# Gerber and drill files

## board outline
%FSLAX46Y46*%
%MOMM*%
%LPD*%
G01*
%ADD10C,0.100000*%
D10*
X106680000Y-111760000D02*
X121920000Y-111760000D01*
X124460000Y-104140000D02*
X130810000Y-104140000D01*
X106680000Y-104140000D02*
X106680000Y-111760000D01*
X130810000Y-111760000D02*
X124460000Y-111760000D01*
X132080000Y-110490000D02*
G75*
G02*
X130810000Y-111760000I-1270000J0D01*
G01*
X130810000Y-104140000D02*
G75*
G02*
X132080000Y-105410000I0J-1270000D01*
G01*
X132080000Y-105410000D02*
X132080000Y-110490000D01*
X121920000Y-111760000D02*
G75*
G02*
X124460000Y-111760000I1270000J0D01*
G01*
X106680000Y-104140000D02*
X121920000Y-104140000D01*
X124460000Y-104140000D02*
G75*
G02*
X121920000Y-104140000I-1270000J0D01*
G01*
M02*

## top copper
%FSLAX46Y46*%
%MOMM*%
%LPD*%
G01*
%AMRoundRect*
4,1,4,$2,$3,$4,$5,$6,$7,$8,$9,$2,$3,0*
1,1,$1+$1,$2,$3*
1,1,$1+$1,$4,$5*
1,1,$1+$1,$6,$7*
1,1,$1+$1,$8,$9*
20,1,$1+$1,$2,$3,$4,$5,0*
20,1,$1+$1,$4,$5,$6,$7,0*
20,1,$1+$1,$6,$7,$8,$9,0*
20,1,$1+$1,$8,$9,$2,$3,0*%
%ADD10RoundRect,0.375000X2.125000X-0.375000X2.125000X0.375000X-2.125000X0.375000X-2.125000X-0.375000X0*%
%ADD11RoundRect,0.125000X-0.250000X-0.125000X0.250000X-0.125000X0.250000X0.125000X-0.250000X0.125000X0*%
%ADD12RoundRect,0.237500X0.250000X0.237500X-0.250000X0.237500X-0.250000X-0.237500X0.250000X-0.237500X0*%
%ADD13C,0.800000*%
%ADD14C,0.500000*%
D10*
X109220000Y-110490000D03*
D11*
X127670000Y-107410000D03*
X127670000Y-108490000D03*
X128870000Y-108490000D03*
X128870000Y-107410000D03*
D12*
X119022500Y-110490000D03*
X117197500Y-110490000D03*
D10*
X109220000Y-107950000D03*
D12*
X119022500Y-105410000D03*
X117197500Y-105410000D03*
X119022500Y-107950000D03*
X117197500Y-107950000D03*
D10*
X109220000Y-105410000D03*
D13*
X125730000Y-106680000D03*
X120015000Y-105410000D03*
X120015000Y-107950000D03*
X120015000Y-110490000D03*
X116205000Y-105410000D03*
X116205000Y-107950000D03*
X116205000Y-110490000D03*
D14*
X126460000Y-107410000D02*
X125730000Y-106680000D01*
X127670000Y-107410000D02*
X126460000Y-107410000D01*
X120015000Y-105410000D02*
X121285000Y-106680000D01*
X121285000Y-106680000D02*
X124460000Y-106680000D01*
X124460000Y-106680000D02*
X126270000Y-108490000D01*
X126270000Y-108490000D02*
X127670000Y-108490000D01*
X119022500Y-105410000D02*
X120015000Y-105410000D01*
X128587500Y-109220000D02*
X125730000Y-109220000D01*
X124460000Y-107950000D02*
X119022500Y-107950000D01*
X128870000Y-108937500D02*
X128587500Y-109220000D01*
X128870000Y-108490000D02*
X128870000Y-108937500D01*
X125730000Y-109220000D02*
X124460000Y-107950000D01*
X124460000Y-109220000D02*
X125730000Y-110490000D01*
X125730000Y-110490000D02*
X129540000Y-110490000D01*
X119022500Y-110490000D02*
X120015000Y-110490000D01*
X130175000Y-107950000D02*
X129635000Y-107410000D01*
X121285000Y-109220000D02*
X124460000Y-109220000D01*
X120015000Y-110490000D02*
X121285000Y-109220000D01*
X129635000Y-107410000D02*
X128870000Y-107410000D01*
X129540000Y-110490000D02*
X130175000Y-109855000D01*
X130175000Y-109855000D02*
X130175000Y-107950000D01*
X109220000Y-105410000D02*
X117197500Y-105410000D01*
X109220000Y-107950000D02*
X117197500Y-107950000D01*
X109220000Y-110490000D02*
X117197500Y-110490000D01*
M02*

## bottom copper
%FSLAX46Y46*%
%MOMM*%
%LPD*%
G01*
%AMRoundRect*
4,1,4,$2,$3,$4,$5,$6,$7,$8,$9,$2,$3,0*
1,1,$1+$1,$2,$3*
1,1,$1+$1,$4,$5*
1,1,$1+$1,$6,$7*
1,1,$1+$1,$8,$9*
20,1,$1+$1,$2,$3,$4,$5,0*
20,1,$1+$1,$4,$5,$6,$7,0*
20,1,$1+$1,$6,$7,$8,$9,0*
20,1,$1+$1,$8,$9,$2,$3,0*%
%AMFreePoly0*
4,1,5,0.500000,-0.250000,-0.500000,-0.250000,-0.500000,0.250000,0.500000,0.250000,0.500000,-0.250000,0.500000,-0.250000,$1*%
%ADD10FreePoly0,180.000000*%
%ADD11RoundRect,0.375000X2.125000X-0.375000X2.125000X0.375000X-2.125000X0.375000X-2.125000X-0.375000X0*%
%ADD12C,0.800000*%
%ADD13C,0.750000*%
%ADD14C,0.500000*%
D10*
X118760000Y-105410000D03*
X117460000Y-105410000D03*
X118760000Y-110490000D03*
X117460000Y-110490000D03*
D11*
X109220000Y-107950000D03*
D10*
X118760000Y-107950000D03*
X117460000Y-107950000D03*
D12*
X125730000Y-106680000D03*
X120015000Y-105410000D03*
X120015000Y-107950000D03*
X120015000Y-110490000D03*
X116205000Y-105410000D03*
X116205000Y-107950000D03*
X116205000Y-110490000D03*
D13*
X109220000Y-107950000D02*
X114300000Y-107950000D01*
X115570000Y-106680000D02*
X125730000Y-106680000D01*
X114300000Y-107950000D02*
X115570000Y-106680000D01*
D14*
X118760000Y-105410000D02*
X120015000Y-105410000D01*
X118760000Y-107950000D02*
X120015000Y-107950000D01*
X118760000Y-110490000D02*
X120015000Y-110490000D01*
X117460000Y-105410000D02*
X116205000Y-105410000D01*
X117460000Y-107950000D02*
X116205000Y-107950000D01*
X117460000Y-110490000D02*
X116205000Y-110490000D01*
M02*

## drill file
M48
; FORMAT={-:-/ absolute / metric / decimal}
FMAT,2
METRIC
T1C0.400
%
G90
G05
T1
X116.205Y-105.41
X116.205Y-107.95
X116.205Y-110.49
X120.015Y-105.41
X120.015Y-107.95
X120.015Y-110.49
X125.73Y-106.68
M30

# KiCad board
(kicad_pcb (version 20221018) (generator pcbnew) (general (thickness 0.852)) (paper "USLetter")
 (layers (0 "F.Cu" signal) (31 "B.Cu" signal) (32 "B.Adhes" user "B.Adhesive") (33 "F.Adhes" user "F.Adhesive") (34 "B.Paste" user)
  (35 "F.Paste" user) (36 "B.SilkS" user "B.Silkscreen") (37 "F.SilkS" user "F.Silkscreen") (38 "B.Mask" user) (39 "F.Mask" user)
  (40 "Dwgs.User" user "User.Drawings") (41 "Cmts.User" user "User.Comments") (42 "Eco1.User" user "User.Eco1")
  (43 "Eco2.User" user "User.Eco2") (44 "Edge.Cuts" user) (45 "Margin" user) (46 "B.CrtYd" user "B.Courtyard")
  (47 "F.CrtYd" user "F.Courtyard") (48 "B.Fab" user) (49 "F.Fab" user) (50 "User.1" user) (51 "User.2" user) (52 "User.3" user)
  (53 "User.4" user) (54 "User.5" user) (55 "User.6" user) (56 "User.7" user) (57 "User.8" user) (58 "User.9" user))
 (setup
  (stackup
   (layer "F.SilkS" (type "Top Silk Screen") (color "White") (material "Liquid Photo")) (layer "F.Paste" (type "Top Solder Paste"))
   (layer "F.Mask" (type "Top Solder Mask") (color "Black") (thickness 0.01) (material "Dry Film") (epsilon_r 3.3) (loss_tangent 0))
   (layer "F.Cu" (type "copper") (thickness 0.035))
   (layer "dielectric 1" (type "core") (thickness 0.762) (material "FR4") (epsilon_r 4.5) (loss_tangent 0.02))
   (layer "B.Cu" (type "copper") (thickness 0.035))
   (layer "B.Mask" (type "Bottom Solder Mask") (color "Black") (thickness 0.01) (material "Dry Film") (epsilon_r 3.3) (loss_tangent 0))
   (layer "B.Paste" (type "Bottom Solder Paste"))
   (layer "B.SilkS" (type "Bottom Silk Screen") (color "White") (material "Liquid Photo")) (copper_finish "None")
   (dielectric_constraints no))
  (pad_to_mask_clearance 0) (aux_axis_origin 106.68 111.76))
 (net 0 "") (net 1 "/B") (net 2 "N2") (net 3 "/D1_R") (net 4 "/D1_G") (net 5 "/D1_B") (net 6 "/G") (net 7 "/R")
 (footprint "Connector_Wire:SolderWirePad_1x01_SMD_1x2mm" (layer "F.Cu") (at 109.22 110.49 90)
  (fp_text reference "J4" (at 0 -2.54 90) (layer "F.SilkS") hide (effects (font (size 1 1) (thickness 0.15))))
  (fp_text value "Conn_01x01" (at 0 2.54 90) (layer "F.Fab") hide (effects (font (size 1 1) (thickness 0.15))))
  (pad "1" smd roundrect (at 0 0 90) (size 1.5 5) (layers "F.Cu" "F.Paste" "F.Mask") (roundrect_rratio 0.25) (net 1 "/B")))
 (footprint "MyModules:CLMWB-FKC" (layer "F.Cu") (at 128.27 107.95)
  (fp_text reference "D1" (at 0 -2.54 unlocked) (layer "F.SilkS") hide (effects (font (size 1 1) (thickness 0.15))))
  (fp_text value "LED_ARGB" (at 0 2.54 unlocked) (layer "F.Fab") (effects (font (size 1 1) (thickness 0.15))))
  (pad "1" smd roundrect (at -0.6 -0.54) (size 0.75 0.5) (layers "F.Cu" "F.Paste" "F.Mask") (roundrect_rratio 0.25) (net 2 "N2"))
  (pad "2" smd roundrect (at -0.6 0.54) (size 0.75 0.5) (layers "F.Cu" "F.Paste" "F.Mask") (roundrect_rratio 0.25) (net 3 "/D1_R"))
  (pad "3" smd roundrect (at 0.6 0.54) (size 0.75 0.5) (layers "F.Cu" "F.Paste" "F.Mask") (roundrect_rratio 0.25) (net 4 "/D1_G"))
  (pad "4" smd roundrect (at 0.6 -0.54) (size 0.75 0.5) (layers "F.Cu" "F.Paste" "F.Mask") (roundrect_rratio 0.25) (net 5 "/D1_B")))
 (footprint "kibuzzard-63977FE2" (layer "F.Cu") (at 113.792 105.41)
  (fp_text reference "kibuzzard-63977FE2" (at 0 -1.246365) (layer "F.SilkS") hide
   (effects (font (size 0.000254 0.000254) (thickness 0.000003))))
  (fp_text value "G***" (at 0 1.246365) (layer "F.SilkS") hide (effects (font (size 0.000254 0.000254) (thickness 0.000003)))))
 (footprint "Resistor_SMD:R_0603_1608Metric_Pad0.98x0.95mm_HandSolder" (layer "F.Cu") (at 118.11 110.49 180)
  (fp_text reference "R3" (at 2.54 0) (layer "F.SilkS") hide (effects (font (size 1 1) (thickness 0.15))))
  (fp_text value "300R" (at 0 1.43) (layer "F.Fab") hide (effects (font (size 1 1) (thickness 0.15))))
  (pad "1" smd roundrect (at -0.9125 0 180) (size 0.975 0.95) (layers "F.Cu" "F.Paste" "F.Mask") (roundrect_rratio 0.25) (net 5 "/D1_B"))
  (pad "2" smd roundrect (at 0.9125 0 180) (size 0.975 0.95) (layers "F.Cu" "F.Paste" "F.Mask") (roundrect_rratio 0.25) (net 1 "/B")))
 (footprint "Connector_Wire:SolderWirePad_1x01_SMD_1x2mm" (layer "F.Cu") (at 109.22 107.95 90)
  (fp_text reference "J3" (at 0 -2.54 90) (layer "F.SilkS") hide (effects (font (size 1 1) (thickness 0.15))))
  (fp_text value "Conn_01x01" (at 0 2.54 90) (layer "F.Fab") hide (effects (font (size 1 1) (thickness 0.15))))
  (pad "1" smd roundrect (at 0 0 90) (size 1.5 5) (layers "F.Cu" "F.Paste" "F.Mask") (roundrect_rratio 0.25) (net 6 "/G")))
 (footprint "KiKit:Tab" (layer "F.Cu") (at 114.046 112.014 90)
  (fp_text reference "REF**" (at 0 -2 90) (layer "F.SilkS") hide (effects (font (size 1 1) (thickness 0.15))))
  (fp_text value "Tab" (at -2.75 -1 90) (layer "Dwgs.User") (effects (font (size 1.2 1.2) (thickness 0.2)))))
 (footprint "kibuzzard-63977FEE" (layer "F.Cu") (at 113.792 107.95)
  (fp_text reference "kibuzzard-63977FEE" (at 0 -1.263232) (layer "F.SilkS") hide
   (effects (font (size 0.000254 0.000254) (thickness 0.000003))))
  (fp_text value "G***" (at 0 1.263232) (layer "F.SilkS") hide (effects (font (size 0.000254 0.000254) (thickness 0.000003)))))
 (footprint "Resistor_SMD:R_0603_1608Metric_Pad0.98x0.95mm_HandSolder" (layer "F.Cu") (at 118.11 105.41 180)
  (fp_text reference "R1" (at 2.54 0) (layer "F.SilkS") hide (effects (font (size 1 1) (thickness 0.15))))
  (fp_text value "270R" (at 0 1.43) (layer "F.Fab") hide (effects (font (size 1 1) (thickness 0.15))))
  (pad "1" smd roundrect (at -0.9125 0 180) (size 0.975 0.95) (layers "F.Cu" "F.Paste" "F.Mask") (roundrect_rratio 0.25) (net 3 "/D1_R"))
  (pad "2" smd roundrect (at 0.9125 0 180) (size 0.975 0.95) (layers "F.Cu" "F.Paste" "F.Mask") (roundrect_rratio 0.25) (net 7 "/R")))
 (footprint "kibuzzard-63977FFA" (layer "F.Cu") (at 113.792 110.49)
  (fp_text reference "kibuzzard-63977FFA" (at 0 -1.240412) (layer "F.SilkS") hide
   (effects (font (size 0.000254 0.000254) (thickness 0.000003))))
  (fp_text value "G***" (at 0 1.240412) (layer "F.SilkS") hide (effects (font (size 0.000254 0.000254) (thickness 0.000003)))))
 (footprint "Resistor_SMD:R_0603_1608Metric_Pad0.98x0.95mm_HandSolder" (layer "F.Cu") (at 118.11 107.95 180)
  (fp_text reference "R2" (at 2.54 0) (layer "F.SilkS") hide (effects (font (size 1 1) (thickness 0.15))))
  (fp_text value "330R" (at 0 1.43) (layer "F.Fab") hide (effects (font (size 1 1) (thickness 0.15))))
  (pad "1" smd roundrect (at -0.9125 0 180) (size 0.975 0.95) (layers "F.Cu" "F.Paste" "F.Mask") (roundrect_rratio 0.25) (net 4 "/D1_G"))
  (pad "2" smd roundrect (at 0.9125 0 180) (size 0.975 0.95) (layers "F.Cu" "F.Paste" "F.Mask") (roundrect_rratio 0.25) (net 6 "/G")))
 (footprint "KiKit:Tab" (layer "F.Cu") (at 114.046 103.886 -90)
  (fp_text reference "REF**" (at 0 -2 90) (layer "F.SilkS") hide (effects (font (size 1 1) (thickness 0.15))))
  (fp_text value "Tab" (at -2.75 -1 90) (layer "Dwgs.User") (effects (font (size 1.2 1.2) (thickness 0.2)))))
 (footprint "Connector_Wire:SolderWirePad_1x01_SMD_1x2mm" (layer "F.Cu") (at 109.22 105.41 90)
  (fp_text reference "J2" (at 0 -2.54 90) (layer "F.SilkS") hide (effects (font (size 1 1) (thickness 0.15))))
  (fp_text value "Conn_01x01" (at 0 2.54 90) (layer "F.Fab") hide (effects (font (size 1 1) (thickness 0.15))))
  (pad "1" smd roundrect (at 0 0 90) (size 1.5 5) (layers "F.Cu" "F.Paste" "F.Mask") (roundrect_rratio 0.25) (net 7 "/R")))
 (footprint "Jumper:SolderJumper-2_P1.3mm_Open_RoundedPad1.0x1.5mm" (layer "B.Cu") (at 118.11 105.41 180)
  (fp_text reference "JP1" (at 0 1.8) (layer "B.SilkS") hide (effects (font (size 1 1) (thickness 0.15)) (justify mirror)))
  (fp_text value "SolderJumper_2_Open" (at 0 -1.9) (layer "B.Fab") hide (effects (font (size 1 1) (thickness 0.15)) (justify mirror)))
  (pad "1" smd custom (at -0.65 0 180) (size 1 0.5) (layers "B.Cu" "B.Mask") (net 3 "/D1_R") (zone_connect 2)
   (options (clearance outline) (anchor rect)) (primitives))
  (pad "2" smd custom (at 0.65 0 180) (size 1 0.5) (layers "B.Cu" "B.Mask") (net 7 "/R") (zone_connect 2)
   (options (clearance outline) (anchor rect)) (primitives)))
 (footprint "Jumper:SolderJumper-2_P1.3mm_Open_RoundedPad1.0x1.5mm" (layer "B.Cu") (at 118.11 110.49 180)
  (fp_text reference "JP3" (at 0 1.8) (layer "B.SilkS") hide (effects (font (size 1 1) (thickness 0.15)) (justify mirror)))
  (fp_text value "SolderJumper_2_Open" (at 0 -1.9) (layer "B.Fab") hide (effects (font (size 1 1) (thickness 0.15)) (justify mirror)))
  (pad "1" smd custom (at -0.65 0 180) (size 1 0.5) (layers "B.Cu" "B.Mask") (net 5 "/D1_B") (zone_connect 2)
   (options (clearance outline) (anchor rect)) (primitives))
  (pad "2" smd custom (at 0.65 0 180) (size 1 0.5) (layers "B.Cu" "B.Mask") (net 1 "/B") (zone_connect 2)
   (options (clearance outline) (anchor rect)) (primitives)))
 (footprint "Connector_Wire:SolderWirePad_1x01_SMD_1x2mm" (layer "B.Cu") (at 109.22 107.95 90)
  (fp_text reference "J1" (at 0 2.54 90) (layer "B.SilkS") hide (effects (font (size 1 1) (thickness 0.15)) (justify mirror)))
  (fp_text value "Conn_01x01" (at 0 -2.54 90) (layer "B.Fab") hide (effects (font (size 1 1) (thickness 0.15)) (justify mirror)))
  (pad "1" smd roundrect (at 0 0 90) (size 1.5 5) (layers "B.Cu" "B.Paste" "B.Mask") (roundrect_rratio 0.25) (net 2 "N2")))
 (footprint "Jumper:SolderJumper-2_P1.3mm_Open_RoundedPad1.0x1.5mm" (layer "B.Cu") (at 118.11 107.95 180)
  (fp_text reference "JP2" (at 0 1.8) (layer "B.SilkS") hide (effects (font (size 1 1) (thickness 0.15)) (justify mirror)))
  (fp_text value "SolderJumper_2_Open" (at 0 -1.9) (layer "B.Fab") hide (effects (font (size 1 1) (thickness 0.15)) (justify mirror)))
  (pad "1" smd custom (at -0.65 0 180) (size 1 0.5) (layers "B.Cu" "B.Mask") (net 4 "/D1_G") (zone_connect 2)
   (options (clearance outline) (anchor rect)) (primitives))
  (pad "2" smd custom (at 0.65 0 180) (size 1 0.5) (layers "B.Cu" "B.Mask") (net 6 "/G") (zone_connect 2)
   (options (clearance outline) (anchor rect)) (primitives)))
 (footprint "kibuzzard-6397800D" (layer "B.Cu") (at 114.046 107.95 180)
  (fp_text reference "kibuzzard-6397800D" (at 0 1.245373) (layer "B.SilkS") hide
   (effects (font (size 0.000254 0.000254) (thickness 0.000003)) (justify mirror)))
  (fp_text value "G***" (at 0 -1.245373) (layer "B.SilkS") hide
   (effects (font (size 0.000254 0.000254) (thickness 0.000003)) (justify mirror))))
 (gr_line (start 106.68 111.76) (end 121.92 111.76) (stroke (width 0.1) (type solid)) (layer "Edge.Cuts"))
 (gr_line (start 124.46 104.14) (end 130.81 104.14) (stroke (width 0.1) (type solid)) (layer "Edge.Cuts"))
 (gr_line (start 106.68 104.14) (end 106.68 111.76) (stroke (width 0.1) (type solid)) (layer "Edge.Cuts"))
 (gr_line (start 130.81 111.76) (end 124.46 111.76) (stroke (width 0.1) (type solid)) (layer "Edge.Cuts"))
 (gr_arc (start 132.08 110.49) (mid 131.708026 111.388026) (end 130.81 111.76) (stroke (width 0.1) (type solid)) (layer "Edge.Cuts"))
 (gr_arc (start 130.81 104.14) (mid 131.708026 104.511974) (end 132.08 105.41) (stroke (width 0.1) (type solid)) (layer "Edge.Cuts"))
 (gr_line (start 132.08 105.41) (end 132.08 110.49) (stroke (width 0.1) (type solid)) (layer "Edge.Cuts"))
 (gr_arc (start 121.92 111.76) (mid 123.19 110.49) (end 124.46 111.76) (stroke (width 0.1) (type solid)) (layer "Edge.Cuts"))
 (gr_line (start 106.68 104.14) (end 121.92 104.14) (stroke (width 0.1) (type solid)) (layer "Edge.Cuts"))
 (gr_arc (start 124.46 104.14) (mid 123.19 105.41) (end 121.92 104.14) (stroke (width 0.1) (type solid)) (layer "Edge.Cuts"))
 (segment (start 126.46 107.41) (end 125.73 106.68) (width 0.5) (layer "F.Cu") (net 2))
 (segment (start 127.67 107.41) (end 126.46 107.41) (width 0.5) (layer "F.Cu") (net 2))
 (via (at 125.73 106.68) (size 0.8) (drill 0.4) (layers "F.Cu" "B.Cu") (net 2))
 (segment (start 109.22 107.95) (end 114.3 107.95) (width 0.75) (layer "B.Cu") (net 2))
 (segment (start 115.57 106.68) (end 125.73 106.68) (width 0.75) (layer "B.Cu") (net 2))
 (segment (start 114.3 107.95) (end 115.57 106.68) (width 0.75) (layer "B.Cu") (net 2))
 (segment (start 120.015 105.41) (end 121.285 106.68) (width 0.5) (layer "F.Cu") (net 3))
 (segment (start 121.285 106.68) (end 124.46 106.68) (width 0.5) (layer "F.Cu") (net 3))
 (segment (start 124.46 106.68) (end 126.27 108.49) (width 0.5) (layer "F.Cu") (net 3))
 (segment (start 126.27 108.49) (end 127.67 108.49) (width 0.5) (layer "F.Cu") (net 3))
 (segment (start 119.0225 105.41) (end 120.015 105.41) (width 0.5) (layer "F.Cu") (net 3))
 (via (at 120.015 105.41) (size 0.8) (drill 0.4) (layers "F.Cu" "B.Cu") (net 3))
 (segment (start 118.76 105.41) (end 120.015 105.41) (width 0.5) (layer "B.Cu") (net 3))
 (segment (start 128.5875 109.22) (end 125.73 109.22) (width 0.5) (layer "F.Cu") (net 4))
 (segment (start 124.46 107.95) (end 119.0225 107.95) (width 0.5) (layer "F.Cu") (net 4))
 (segment (start 128.87 108.9375) (end 128.5875 109.22) (width 0.5) (layer "F.Cu") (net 4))
 (segment (start 128.87 108.49) (end 128.87 108.9375) (width 0.5) (layer "F.Cu") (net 4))
 (segment (start 125.73 109.22) (end 124.46 107.95) (width 0.5) (layer "F.Cu") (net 4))
 (via (at 120.015 107.95) (size 0.8) (drill 0.4) (layers "F.Cu" "B.Cu") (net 4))
 (segment (start 118.76 107.95) (end 120.015 107.95) (width 0.5) (layer "B.Cu") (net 4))
 (segment (start 124.46 109.22) (end 125.73 110.49) (width 0.5) (layer "F.Cu") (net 5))
 (segment (start 125.73 110.49) (end 129.54 110.49) (width 0.5) (layer "F.Cu") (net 5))
 (segment (start 119.0225 110.49) (end 120.015 110.49) (width 0.5) (layer "F.Cu") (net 5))
 (segment (start 130.175 107.95) (end 129.635 107.41) (width 0.5) (layer "F.Cu") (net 5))
 (segment (start 121.285 109.22) (end 124.46 109.22) (width 0.5) (layer "F.Cu") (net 5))
 (segment (start 120.015 110.49) (end 121.285 109.22) (width 0.5) (layer "F.Cu") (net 5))
 (segment (start 129.635 107.41) (end 128.87 107.41) (width 0.5) (layer "F.Cu") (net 5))
 (segment (start 129.54 110.49) (end 130.175 109.855) (width 0.5) (layer "F.Cu") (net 5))
 (segment (start 130.175 109.855) (end 130.175 107.95) (width 0.5) (layer "F.Cu") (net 5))
 (via (at 120.015 110.49) (size 0.8) (drill 0.4) (layers "F.Cu" "B.Cu") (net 5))
 (segment (start 118.76 110.49) (end 120.015 110.49) (width 0.5) (layer "B.Cu") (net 5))
 (segment (start 109.22 105.41) (end 117.1975 105.41) (width 0.5) (layer "F.Cu") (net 7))
 (via (at 116.205 105.41) (size 0.8) (drill 0.4) (layers "F.Cu" "B.Cu") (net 7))
 (segment (start 117.46 105.41) (end 116.205 105.41) (width 0.5) (layer "B.Cu") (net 7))
 (segment (start 109.22 107.95) (end 117.1975 107.95) (width 0.5) (layer "F.Cu") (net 6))
 (via (at 116.205 107.95) (size 0.8) (drill 0.4) (layers "F.Cu" "B.Cu") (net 6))
 (segment (start 117.46 107.95) (end 116.205 107.95) (width 0.5) (layer "B.Cu") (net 6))
 (segment (start 109.22 110.49) (end 117.1975 110.49) (width 0.5) (layer "F.Cu") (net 1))
 (via (at 116.205 110.49) (size 0.8) (drill 0.4) (layers "F.Cu" "B.Cu") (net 1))
 (segment (start 117.46 110.49) (end 116.205 110.49) (width 0.5) (layer "B.Cu") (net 1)))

